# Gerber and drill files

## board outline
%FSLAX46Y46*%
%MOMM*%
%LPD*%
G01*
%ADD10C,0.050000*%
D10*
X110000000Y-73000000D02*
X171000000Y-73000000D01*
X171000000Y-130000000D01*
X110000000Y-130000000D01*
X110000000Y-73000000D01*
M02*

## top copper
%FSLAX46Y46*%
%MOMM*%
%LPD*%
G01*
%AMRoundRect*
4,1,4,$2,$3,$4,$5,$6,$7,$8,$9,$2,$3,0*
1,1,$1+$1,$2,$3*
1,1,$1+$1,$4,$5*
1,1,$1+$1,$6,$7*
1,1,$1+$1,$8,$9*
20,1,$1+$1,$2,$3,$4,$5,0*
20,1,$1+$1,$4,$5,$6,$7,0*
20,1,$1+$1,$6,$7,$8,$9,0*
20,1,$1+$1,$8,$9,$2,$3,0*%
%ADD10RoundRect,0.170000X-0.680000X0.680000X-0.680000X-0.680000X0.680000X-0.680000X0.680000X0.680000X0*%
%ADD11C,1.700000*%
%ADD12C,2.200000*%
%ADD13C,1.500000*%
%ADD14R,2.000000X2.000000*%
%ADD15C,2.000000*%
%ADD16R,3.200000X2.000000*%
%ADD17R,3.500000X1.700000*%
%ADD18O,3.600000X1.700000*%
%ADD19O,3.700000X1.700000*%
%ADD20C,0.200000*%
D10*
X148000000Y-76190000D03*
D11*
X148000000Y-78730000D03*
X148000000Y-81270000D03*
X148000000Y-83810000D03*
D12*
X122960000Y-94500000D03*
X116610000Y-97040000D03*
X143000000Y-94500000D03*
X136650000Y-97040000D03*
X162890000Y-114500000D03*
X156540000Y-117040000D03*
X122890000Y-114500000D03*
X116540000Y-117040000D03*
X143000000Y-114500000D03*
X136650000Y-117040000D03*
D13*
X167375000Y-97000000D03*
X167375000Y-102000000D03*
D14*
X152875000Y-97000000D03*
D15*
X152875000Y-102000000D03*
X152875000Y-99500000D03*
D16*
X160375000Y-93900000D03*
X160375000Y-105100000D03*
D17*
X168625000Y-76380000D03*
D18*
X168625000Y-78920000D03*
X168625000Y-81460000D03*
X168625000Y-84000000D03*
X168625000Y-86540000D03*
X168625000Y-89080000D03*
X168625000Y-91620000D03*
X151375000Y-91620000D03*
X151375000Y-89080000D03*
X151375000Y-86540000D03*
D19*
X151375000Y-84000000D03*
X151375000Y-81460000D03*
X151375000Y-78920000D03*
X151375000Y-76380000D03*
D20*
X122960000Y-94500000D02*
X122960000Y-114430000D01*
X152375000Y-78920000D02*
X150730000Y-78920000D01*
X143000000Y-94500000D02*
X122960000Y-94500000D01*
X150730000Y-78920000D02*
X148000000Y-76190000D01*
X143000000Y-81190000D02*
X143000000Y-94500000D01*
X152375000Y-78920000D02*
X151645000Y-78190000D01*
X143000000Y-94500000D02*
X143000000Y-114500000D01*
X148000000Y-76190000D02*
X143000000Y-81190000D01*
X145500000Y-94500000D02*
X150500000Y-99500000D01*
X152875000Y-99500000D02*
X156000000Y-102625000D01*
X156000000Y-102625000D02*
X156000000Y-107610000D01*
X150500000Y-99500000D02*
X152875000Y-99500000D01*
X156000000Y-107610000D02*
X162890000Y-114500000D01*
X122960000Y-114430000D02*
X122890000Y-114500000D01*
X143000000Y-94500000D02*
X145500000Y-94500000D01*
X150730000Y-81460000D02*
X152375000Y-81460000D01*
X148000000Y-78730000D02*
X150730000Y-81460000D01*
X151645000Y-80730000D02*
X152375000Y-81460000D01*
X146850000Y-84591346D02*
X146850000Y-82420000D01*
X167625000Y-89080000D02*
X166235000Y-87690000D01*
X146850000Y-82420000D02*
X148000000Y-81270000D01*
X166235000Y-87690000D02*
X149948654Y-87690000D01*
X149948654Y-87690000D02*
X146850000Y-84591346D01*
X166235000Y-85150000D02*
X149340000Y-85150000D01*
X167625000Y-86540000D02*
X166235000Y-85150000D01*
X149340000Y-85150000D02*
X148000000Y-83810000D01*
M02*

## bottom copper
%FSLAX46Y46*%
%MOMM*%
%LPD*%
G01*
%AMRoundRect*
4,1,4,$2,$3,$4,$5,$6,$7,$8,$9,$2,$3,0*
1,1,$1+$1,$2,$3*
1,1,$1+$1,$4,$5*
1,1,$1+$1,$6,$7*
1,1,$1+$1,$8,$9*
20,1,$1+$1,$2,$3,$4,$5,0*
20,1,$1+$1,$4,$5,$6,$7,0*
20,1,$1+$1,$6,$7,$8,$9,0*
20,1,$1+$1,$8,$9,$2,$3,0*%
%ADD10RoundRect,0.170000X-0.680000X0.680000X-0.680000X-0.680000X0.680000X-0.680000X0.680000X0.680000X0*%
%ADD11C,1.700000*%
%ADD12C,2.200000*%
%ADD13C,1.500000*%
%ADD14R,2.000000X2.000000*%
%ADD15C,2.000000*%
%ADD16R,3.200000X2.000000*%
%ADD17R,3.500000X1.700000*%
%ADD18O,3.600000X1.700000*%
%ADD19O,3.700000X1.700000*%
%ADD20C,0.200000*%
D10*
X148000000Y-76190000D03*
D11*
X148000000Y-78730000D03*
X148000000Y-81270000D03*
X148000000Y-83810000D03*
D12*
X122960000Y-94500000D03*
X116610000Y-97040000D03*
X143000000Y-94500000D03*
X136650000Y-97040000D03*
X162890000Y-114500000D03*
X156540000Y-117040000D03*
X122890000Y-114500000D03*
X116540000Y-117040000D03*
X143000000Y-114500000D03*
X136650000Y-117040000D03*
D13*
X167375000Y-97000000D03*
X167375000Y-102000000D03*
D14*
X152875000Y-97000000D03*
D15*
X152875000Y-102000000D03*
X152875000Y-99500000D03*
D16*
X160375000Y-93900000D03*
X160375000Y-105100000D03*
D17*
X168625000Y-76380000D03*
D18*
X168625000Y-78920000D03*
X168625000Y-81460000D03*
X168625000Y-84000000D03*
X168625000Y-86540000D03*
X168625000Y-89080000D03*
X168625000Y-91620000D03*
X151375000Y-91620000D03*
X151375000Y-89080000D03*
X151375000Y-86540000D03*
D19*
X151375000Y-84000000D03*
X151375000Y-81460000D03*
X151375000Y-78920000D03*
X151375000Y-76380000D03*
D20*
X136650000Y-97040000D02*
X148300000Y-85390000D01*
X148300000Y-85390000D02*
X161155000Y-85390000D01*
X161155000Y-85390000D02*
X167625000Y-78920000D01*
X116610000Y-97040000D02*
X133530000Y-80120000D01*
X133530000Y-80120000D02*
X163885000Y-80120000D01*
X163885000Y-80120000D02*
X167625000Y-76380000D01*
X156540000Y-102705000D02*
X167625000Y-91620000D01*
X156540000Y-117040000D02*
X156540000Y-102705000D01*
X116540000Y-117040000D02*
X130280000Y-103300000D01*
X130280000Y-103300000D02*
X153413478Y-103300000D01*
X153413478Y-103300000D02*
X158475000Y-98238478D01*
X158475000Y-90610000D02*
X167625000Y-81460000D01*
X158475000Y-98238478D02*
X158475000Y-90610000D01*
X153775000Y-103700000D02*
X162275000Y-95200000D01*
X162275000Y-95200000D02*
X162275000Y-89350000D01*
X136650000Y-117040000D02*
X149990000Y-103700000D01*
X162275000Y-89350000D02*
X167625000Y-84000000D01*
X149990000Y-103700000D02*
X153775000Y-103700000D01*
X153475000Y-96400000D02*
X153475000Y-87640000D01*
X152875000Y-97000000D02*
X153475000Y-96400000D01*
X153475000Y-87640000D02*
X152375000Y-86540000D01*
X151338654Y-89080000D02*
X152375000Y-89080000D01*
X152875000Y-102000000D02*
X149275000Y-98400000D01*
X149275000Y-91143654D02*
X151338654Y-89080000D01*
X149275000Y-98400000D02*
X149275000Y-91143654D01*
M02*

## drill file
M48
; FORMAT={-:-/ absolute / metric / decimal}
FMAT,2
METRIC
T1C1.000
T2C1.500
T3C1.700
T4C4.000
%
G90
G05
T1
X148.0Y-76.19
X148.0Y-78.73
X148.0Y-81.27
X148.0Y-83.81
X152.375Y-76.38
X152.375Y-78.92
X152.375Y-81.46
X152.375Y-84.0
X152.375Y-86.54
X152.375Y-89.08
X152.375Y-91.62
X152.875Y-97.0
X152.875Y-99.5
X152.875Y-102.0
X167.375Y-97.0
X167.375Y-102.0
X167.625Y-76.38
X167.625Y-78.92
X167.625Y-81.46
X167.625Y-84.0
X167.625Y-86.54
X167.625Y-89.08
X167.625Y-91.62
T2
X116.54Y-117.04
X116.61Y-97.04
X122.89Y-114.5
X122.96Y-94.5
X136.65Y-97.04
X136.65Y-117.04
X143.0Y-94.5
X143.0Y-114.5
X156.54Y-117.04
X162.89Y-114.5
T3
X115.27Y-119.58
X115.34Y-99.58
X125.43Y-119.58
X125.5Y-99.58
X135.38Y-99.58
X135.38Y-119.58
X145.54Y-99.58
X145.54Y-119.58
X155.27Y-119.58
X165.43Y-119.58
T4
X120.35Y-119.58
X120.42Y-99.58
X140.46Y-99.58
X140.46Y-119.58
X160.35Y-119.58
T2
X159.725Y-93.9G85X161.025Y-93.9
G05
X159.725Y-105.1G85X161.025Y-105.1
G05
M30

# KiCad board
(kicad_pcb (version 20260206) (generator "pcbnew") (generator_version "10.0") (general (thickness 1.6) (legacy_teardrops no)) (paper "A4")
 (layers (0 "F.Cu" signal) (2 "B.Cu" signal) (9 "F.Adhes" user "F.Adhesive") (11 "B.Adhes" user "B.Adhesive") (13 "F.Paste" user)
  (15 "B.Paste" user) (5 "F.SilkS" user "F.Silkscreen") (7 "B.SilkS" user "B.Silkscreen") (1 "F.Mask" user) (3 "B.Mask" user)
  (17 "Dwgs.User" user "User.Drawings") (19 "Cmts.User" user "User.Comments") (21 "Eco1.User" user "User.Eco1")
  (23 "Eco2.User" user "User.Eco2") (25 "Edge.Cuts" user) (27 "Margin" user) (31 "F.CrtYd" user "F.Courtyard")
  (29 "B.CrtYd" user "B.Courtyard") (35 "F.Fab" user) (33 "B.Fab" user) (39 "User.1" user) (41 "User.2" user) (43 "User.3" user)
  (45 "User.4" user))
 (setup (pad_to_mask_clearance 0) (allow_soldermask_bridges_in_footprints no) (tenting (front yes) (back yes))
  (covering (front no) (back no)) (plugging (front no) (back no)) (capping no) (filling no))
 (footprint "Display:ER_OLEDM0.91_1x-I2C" (layer "F.Cu") (at 148 76.19 -90)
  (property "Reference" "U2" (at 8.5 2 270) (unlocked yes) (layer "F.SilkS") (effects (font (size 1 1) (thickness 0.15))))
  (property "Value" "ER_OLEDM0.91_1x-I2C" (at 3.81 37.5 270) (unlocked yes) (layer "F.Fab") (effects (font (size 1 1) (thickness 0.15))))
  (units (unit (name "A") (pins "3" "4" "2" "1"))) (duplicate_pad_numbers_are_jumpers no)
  (pad "1" thru_hole roundrect (at 0 0 270) (size 1.7 1.7) (drill 1) (layers "*.Cu" "*.Mask") (remove_unused_layers no)
   (roundrect_rratio 0.1) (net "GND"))
  (pad "2" thru_hole circle (at 2.54 0 270) (size 1.7 1.7) (drill 1) (layers "*.Cu" "*.Mask") (remove_unused_layers no) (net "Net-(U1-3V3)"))
  (pad "3" thru_hole circle (at 5.08 0 270) (size 1.7 1.7) (drill 1) (layers "*.Cu" "*.Mask") (remove_unused_layers no)
   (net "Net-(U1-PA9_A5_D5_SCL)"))
  (pad "4" thru_hole circle (at 7.62 0 270) (size 1.7 1.7) (drill 1) (layers "*.Cu" "*.Mask") (remove_unused_layers no)
   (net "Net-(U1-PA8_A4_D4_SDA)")))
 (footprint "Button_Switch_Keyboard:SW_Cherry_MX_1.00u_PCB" (layer "F.Cu") (at 122.96 94.5)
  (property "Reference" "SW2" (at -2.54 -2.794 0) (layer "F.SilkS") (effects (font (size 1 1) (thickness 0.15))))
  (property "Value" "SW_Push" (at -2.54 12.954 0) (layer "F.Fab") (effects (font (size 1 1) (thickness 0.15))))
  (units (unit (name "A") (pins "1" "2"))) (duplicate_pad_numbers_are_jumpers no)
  (pad "" np_thru_hole circle (at -7.62 5.08) (size 1.7 1.7) (drill 1.7) (layers "*.Cu" "*.Mask"))
  (pad "" np_thru_hole circle (at -2.54 5.08) (size 4 4) (drill 4) (layers "*.Cu" "*.Mask"))
  (pad "" np_thru_hole circle (at 2.54 5.08) (size 1.7 1.7) (drill 1.7) (layers "*.Cu" "*.Mask"))
  (pad "1" thru_hole circle (at 0 0) (size 2.2 2.2) (drill 1.5) (layers "*.Cu" "*.Mask") (remove_unused_layers no) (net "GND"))
  (pad "2" thru_hole circle (at -6.35 2.54) (size 2.2 2.2) (drill 1.5) (layers "*.Cu" "*.Mask") (remove_unused_layers no)
   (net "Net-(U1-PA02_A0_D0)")))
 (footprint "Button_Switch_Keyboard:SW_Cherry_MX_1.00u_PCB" (layer "F.Cu") (at 143 94.5)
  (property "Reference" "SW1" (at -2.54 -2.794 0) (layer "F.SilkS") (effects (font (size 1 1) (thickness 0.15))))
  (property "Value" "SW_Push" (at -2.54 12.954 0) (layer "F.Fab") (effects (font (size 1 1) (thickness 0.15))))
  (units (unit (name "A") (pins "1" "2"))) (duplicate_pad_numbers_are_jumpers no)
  (pad "" np_thru_hole circle (at -7.62 5.08) (size 1.7 1.7) (drill 1.7) (layers "*.Cu" "*.Mask"))
  (pad "" np_thru_hole circle (at -2.54 5.08) (size 4 4) (drill 4) (layers "*.Cu" "*.Mask"))
  (pad "" np_thru_hole circle (at 2.54 5.08) (size 1.7 1.7) (drill 1.7) (layers "*.Cu" "*.Mask"))
  (pad "1" thru_hole circle (at 0 0) (size 2.2 2.2) (drill 1.5) (layers "*.Cu" "*.Mask") (remove_unused_layers no) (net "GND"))
  (pad "2" thru_hole circle (at -6.35 2.54) (size 2.2 2.2) (drill 1.5) (layers "*.Cu" "*.Mask") (remove_unused_layers no)
   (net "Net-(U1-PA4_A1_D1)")))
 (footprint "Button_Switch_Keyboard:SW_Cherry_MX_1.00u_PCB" (layer "F.Cu") (at 162.89 114.5)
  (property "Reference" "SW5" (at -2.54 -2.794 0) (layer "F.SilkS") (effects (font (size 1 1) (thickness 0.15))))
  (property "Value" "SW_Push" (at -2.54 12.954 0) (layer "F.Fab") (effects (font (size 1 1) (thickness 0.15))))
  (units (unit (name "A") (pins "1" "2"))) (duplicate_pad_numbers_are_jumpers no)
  (pad "" np_thru_hole circle (at -7.62 5.08) (size 1.7 1.7) (drill 1.7) (layers "*.Cu" "*.Mask"))
  (pad "" np_thru_hole circle (at -2.54 5.08) (size 4 4) (drill 4) (layers "*.Cu" "*.Mask"))
  (pad "" np_thru_hole circle (at 2.54 5.08) (size 1.7 1.7) (drill 1.7) (layers "*.Cu" "*.Mask"))
  (pad "1" thru_hole circle (at 0 0) (size 2.2 2.2) (drill 1.5) (layers "*.Cu" "*.Mask") (remove_unused_layers no) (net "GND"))
  (pad "2" thru_hole circle (at -6.35 2.54) (size 2.2 2.2) (drill 1.5) (layers "*.Cu" "*.Mask") (remove_unused_layers no)
   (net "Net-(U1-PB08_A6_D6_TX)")))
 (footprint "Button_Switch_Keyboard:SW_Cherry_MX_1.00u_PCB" (layer "F.Cu") (at 122.89 114.5)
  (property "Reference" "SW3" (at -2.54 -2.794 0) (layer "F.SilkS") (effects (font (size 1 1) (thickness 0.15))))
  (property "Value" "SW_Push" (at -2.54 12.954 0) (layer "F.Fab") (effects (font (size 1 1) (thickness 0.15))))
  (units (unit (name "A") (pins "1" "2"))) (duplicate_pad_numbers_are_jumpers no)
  (pad "" np_thru_hole circle (at -7.62 5.08) (size 1.7 1.7) (drill 1.7) (layers "*.Cu" "*.Mask"))
  (pad "" np_thru_hole circle (at -2.54 5.08) (size 4 4) (drill 4) (layers "*.Cu" "*.Mask"))
  (pad "" np_thru_hole circle (at 2.54 5.08) (size 1.7 1.7) (drill 1.7) (layers "*.Cu" "*.Mask"))
  (pad "1" thru_hole circle (at 0 0) (size 2.2 2.2) (drill 1.5) (layers "*.Cu" "*.Mask") (remove_unused_layers no) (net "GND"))
  (pad "2" thru_hole circle (at -6.35 2.54) (size 2.2 2.2) (drill 1.5) (layers "*.Cu" "*.Mask") (remove_unused_layers no)
   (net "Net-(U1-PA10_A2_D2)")))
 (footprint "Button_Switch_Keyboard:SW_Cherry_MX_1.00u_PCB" (layer "F.Cu") (at 143 114.5)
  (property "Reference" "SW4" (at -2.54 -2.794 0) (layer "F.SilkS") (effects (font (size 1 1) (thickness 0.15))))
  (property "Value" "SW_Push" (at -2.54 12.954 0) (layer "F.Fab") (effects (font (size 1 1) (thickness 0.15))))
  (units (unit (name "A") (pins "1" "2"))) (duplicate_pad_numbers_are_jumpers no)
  (pad "" np_thru_hole circle (at -7.62 5.08) (size 1.7 1.7) (drill 1.7) (layers "*.Cu" "*.Mask"))
  (pad "" np_thru_hole circle (at -2.54 5.08) (size 4 4) (drill 4) (layers "*.Cu" "*.Mask"))
  (pad "" np_thru_hole circle (at 2.54 5.08) (size 1.7 1.7) (drill 1.7) (layers "*.Cu" "*.Mask"))
  (pad "1" thru_hole circle (at 0 0) (size 2.2 2.2) (drill 1.5) (layers "*.Cu" "*.Mask") (remove_unused_layers no) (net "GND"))
  (pad "2" thru_hole circle (at -6.35 2.54) (size 2.2 2.2) (drill 1.5) (layers "*.Cu" "*.Mask") (remove_unused_layers no)
   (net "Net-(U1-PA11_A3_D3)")))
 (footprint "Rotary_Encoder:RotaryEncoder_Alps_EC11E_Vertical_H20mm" (layer "F.Cu") (at 152.875 97)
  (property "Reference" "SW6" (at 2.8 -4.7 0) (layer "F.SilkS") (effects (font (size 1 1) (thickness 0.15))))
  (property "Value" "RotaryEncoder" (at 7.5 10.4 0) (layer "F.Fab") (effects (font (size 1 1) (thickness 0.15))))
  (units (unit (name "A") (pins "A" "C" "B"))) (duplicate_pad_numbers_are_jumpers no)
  (pad "" thru_hole circle (at 14.5 0) (size 1.5 1.5) (drill 1) (layers "*.Cu" "*.Mask") (remove_unused_layers no))
  (pad "" thru_hole circle (at 14.5 5) (size 1.5 1.5) (drill 1) (layers "*.Cu" "*.Mask") (remove_unused_layers no))
  (pad "A" thru_hole rect (at 0 0) (size 2 2) (drill 1) (layers "*.Cu" "*.Mask") (remove_unused_layers no) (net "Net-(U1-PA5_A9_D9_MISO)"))
  (pad "B" thru_hole circle (at 0 5) (size 2 2) (drill 1) (layers "*.Cu" "*.Mask") (remove_unused_layers no) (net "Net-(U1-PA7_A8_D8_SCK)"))
  (pad "C" thru_hole circle (at 0 2.5) (size 2 2) (drill 1) (layers "*.Cu" "*.Mask") (remove_unused_layers no) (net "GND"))
  (pad "MP" thru_hole rect (at 7.5 -3.1) (size 3.2 2) (drill oval 2.8 1.5) (layers "*.Cu" "*.Mask") (remove_unused_layers no))
  (pad "MP" thru_hole rect (at 7.5 8.1) (size 3.2 2) (drill oval 2.8 1.5) (layers "*.Cu" "*.Mask") (remove_unused_layers no)))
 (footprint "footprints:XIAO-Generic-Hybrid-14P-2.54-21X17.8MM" (layer "B.Cu") (at 160 84 180)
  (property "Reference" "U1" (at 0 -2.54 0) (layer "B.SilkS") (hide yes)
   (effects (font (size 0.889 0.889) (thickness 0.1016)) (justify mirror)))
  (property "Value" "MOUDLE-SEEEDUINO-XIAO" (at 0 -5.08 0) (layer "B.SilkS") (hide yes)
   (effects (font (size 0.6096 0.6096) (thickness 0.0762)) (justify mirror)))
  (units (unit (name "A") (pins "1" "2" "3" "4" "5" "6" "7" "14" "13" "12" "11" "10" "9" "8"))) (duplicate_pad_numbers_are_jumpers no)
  (pad "1" thru_hole rect (at -7.625 7.62 180) (size 3.5 1.7) (drill 1 (offset -1 0)) (layers "*.Cu" "*.Mask") (remove_unused_layers no)
   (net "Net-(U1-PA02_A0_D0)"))
  (pad "2" thru_hole oval (at -7.625 5.08 180) (size 3.6 1.7) (drill 1 (offset -1 0)) (layers "*.Cu" "*.Mask") (remove_unused_layers no)
   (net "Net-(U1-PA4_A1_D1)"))
  (pad "3" thru_hole oval (at -7.625 2.54 180) (size 3.6 1.7) (drill 1 (offset -1 0)) (layers "*.Cu" "*.Mask") (remove_unused_layers no)
   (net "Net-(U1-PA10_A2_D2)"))
  (pad "4" thru_hole oval (at -7.625 0 180) (size 3.6 1.7) (drill 1 (offset -1 0)) (layers "*.Cu" "*.Mask") (remove_unused_layers no)
   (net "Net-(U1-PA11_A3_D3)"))
  (pad "5" thru_hole oval (at -7.625 -2.54 180) (size 3.6 1.7) (drill 1 (offset -1 0)) (layers "*.Cu" "*.Mask") (remove_unused_layers no)
   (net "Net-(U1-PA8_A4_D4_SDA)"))
  (pad "6" thru_hole oval (at -7.625 -5.08) (size 3.6 1.7) (drill 1 (offset 1 0)) (layers "*.Cu" "*.Mask") (remove_unused_layers no)
   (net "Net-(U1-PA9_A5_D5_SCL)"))
  (pad "7" thru_hole oval (at -7.625 -7.62 180) (size 3.6 1.7) (drill 1 (offset -1 0)) (layers "*.Cu" "*.Mask") (remove_unused_layers no)
   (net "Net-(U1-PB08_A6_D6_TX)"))
  (pad "8" thru_hole oval (at 7.625 -7.62 180) (size 3.6 1.7) (drill 1 (offset 1 0)) (layers "*.Cu" "*.Mask") (remove_unused_layers no)
   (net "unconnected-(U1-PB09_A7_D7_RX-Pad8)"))
  (pad "9" thru_hole oval (at 7.625 -5.08 180) (size 3.6 1.7) (drill 1 (offset 1 0)) (layers "*.Cu" "*.Mask") (remove_unused_layers no)
   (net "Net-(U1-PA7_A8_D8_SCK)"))
  (pad "10" thru_hole oval (at 7.625 -2.54 180) (size 3.6 1.7) (drill 1 (offset 1 0)) (layers "*.Cu" "*.Mask") (remove_unused_layers no)
   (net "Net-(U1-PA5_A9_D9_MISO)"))
  (pad "11" thru_hole oval (at 7.625 0 180) (size 3.7 1.7) (drill 1 (offset 1 0)) (layers "*.Cu" "*.Mask") (remove_unused_layers no)
   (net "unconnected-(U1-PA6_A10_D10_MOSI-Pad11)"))
  (pad "12" thru_hole oval (at 7.625 2.54 180) (size 3.7 1.7) (drill 1 (offset 1 0)) (layers "*.Cu" "*.Mask") (remove_unused_layers no)
   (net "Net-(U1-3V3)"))
  (pad "13" thru_hole oval (at 7.625 5.08 180) (size 3.7 1.7) (drill 1 (offset 1 0)) (layers "*.Cu" "*.Mask") (remove_unused_layers no)
   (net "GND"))
  (pad "14" thru_hole oval (at 7.625 7.62 180) (size 3.7 1.7) (drill 1 (offset 1 0)) (layers "*.Cu" "*.Mask") (remove_unused_layers no)
   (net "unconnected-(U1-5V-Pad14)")))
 (gr_rect (start 110 73) (end 171 130) (stroke (width 0.05) (type default)) (fill no) (layer "Edge.Cuts"))
 (segment (start 122.96 94.5) (end 122.96 114.43) (width 0.2) (layer "F.Cu") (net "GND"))
 (segment (start 152.375 78.92) (end 150.73 78.92) (width 0.2) (layer "F.Cu") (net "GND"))
 (segment (start 143 94.5) (end 122.96 94.5) (width 0.2) (layer "F.Cu") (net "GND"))
 (segment (start 150.73 78.92) (end 148 76.19) (width 0.2) (layer "F.Cu") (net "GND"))
 (segment (start 143 81.19) (end 143 94.5) (width 0.2) (layer "F.Cu") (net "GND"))
 (segment (start 152.375 78.92) (end 151.645 78.19) (width 0.2) (layer "F.Cu") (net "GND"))
 (segment (start 143 94.5) (end 143 114.5) (width 0.2) (layer "F.Cu") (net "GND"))
 (segment (start 148 76.19) (end 143 81.19) (width 0.2) (layer "F.Cu") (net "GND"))
 (segment (start 145.5 94.5) (end 150.5 99.5) (width 0.2) (layer "F.Cu") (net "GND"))
 (segment (start 152.875 99.5) (end 156 102.625) (width 0.2) (layer "F.Cu") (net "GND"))
 (segment (start 156 102.625) (end 156 107.61) (width 0.2) (layer "F.Cu") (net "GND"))
 (segment (start 150.5 99.5) (end 152.875 99.5) (width 0.2) (layer "F.Cu") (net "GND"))
 (segment (start 156 107.61) (end 162.89 114.5) (width 0.2) (layer "F.Cu") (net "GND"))
 (segment (start 122.96 114.43) (end 122.89 114.5) (width 0.2) (layer "F.Cu") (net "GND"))
 (segment (start 143 94.5) (end 145.5 94.5) (width 0.2) (layer "F.Cu") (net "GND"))
 (segment (start 150.73 81.46) (end 152.375 81.46) (width 0.2) (layer "F.Cu") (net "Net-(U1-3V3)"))
 (segment (start 148 78.73) (end 150.73 81.46) (width 0.2) (layer "F.Cu") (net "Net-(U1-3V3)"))
 (segment (start 151.645 80.73) (end 152.375 81.46) (width 0.2) (layer "F.Cu") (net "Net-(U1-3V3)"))
 (segment (start 146.85 84.591346) (end 146.85 82.42) (width 0.2) (layer "F.Cu") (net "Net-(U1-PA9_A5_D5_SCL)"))
 (segment (start 167.625 89.08) (end 166.235 87.69) (width 0.2) (layer "F.Cu") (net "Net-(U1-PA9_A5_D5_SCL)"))
 (segment (start 146.85 82.42) (end 148 81.27) (width 0.2) (layer "F.Cu") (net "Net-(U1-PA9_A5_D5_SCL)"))
 (segment (start 166.235 87.69) (end 149.948654 87.69) (width 0.2) (layer "F.Cu") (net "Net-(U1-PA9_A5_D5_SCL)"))
 (segment (start 149.948654 87.69) (end 146.85 84.591346) (width 0.2) (layer "F.Cu") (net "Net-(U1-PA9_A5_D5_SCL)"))
 (segment (start 166.235 85.15) (end 149.34 85.15) (width 0.2) (layer "F.Cu") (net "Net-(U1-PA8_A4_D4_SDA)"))
 (segment (start 167.625 86.54) (end 166.235 85.15) (width 0.2) (layer "F.Cu") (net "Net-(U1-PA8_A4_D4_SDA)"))
 (segment (start 149.34 85.15) (end 148 83.81) (width 0.2) (layer "F.Cu") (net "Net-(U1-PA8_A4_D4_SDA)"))
 (segment (start 136.65 97.04) (end 148.3 85.39) (width 0.2) (layer "B.Cu") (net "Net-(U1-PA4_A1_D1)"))
 (segment (start 148.3 85.39) (end 161.155 85.39) (width 0.2) (layer "B.Cu") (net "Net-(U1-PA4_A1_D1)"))
 (segment (start 161.155 85.39) (end 167.625 78.92) (width 0.2) (layer "B.Cu") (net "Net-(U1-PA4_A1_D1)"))
 (segment (start 116.61 97.04) (end 133.53 80.12) (width 0.2) (layer "B.Cu") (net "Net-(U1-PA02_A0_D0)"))
 (segment (start 133.53 80.12) (end 163.885 80.12) (width 0.2) (layer "B.Cu") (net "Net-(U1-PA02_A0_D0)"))
 (segment (start 163.885 80.12) (end 167.625 76.38) (width 0.2) (layer "B.Cu") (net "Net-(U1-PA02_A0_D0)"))
 (segment (start 156.54 102.705) (end 167.625 91.62) (width 0.2) (layer "B.Cu") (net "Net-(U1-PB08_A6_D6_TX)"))
 (segment (start 156.54 117.04) (end 156.54 102.705) (width 0.2) (layer "B.Cu") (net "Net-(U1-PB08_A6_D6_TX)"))
 (segment (start 116.54 117.04) (end 130.28 103.3) (width 0.2) (layer "B.Cu") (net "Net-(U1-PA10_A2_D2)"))
 (segment (start 130.28 103.3) (end 153.413478 103.3) (width 0.2) (layer "B.Cu") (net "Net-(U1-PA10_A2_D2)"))
 (segment (start 153.413478 103.3) (end 158.475 98.238478) (width 0.2) (layer "B.Cu") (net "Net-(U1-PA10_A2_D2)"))
 (segment (start 158.475 90.61) (end 167.625 81.46) (width 0.2) (layer "B.Cu") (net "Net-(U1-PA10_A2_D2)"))
 (segment (start 158.475 98.238478) (end 158.475 90.61) (width 0.2) (layer "B.Cu") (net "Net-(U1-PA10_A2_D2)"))
 (segment (start 153.775 103.7) (end 162.275 95.2) (width 0.2) (layer "B.Cu") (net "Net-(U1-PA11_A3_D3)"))
 (segment (start 162.275 95.2) (end 162.275 89.35) (width 0.2) (layer "B.Cu") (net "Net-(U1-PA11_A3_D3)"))
 (segment (start 136.65 117.04) (end 149.99 103.7) (width 0.2) (layer "B.Cu") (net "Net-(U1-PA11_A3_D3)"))
 (segment (start 162.275 89.35) (end 167.625 84) (width 0.2) (layer "B.Cu") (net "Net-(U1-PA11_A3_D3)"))
 (segment (start 149.99 103.7) (end 153.775 103.7) (width 0.2) (layer "B.Cu") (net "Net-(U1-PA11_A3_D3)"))
 (segment (start 153.475 96.4) (end 153.475 87.64) (width 0.2) (layer "B.Cu") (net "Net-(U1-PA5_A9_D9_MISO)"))
 (segment (start 152.875 97) (end 153.475 96.4) (width 0.2) (layer "B.Cu") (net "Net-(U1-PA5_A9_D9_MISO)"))
 (segment (start 153.475 87.64) (end 152.375 86.54) (width 0.2) (layer "B.Cu") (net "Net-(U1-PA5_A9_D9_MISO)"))
 (segment (start 151.338654 89.08) (end 152.375 89.08) (width 0.2) (layer "B.Cu") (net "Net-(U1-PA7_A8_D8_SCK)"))
 (segment (start 152.875 102) (end 149.275 98.4) (width 0.2) (layer "B.Cu") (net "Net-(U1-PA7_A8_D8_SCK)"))
 (segment (start 149.275 91.143654) (end 151.338654 89.08) (width 0.2) (layer "B.Cu") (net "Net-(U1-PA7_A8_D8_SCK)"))
 (segment (start 149.275 98.4) (end 149.275 91.143654) (width 0.2) (layer "B.Cu") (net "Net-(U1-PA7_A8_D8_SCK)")))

